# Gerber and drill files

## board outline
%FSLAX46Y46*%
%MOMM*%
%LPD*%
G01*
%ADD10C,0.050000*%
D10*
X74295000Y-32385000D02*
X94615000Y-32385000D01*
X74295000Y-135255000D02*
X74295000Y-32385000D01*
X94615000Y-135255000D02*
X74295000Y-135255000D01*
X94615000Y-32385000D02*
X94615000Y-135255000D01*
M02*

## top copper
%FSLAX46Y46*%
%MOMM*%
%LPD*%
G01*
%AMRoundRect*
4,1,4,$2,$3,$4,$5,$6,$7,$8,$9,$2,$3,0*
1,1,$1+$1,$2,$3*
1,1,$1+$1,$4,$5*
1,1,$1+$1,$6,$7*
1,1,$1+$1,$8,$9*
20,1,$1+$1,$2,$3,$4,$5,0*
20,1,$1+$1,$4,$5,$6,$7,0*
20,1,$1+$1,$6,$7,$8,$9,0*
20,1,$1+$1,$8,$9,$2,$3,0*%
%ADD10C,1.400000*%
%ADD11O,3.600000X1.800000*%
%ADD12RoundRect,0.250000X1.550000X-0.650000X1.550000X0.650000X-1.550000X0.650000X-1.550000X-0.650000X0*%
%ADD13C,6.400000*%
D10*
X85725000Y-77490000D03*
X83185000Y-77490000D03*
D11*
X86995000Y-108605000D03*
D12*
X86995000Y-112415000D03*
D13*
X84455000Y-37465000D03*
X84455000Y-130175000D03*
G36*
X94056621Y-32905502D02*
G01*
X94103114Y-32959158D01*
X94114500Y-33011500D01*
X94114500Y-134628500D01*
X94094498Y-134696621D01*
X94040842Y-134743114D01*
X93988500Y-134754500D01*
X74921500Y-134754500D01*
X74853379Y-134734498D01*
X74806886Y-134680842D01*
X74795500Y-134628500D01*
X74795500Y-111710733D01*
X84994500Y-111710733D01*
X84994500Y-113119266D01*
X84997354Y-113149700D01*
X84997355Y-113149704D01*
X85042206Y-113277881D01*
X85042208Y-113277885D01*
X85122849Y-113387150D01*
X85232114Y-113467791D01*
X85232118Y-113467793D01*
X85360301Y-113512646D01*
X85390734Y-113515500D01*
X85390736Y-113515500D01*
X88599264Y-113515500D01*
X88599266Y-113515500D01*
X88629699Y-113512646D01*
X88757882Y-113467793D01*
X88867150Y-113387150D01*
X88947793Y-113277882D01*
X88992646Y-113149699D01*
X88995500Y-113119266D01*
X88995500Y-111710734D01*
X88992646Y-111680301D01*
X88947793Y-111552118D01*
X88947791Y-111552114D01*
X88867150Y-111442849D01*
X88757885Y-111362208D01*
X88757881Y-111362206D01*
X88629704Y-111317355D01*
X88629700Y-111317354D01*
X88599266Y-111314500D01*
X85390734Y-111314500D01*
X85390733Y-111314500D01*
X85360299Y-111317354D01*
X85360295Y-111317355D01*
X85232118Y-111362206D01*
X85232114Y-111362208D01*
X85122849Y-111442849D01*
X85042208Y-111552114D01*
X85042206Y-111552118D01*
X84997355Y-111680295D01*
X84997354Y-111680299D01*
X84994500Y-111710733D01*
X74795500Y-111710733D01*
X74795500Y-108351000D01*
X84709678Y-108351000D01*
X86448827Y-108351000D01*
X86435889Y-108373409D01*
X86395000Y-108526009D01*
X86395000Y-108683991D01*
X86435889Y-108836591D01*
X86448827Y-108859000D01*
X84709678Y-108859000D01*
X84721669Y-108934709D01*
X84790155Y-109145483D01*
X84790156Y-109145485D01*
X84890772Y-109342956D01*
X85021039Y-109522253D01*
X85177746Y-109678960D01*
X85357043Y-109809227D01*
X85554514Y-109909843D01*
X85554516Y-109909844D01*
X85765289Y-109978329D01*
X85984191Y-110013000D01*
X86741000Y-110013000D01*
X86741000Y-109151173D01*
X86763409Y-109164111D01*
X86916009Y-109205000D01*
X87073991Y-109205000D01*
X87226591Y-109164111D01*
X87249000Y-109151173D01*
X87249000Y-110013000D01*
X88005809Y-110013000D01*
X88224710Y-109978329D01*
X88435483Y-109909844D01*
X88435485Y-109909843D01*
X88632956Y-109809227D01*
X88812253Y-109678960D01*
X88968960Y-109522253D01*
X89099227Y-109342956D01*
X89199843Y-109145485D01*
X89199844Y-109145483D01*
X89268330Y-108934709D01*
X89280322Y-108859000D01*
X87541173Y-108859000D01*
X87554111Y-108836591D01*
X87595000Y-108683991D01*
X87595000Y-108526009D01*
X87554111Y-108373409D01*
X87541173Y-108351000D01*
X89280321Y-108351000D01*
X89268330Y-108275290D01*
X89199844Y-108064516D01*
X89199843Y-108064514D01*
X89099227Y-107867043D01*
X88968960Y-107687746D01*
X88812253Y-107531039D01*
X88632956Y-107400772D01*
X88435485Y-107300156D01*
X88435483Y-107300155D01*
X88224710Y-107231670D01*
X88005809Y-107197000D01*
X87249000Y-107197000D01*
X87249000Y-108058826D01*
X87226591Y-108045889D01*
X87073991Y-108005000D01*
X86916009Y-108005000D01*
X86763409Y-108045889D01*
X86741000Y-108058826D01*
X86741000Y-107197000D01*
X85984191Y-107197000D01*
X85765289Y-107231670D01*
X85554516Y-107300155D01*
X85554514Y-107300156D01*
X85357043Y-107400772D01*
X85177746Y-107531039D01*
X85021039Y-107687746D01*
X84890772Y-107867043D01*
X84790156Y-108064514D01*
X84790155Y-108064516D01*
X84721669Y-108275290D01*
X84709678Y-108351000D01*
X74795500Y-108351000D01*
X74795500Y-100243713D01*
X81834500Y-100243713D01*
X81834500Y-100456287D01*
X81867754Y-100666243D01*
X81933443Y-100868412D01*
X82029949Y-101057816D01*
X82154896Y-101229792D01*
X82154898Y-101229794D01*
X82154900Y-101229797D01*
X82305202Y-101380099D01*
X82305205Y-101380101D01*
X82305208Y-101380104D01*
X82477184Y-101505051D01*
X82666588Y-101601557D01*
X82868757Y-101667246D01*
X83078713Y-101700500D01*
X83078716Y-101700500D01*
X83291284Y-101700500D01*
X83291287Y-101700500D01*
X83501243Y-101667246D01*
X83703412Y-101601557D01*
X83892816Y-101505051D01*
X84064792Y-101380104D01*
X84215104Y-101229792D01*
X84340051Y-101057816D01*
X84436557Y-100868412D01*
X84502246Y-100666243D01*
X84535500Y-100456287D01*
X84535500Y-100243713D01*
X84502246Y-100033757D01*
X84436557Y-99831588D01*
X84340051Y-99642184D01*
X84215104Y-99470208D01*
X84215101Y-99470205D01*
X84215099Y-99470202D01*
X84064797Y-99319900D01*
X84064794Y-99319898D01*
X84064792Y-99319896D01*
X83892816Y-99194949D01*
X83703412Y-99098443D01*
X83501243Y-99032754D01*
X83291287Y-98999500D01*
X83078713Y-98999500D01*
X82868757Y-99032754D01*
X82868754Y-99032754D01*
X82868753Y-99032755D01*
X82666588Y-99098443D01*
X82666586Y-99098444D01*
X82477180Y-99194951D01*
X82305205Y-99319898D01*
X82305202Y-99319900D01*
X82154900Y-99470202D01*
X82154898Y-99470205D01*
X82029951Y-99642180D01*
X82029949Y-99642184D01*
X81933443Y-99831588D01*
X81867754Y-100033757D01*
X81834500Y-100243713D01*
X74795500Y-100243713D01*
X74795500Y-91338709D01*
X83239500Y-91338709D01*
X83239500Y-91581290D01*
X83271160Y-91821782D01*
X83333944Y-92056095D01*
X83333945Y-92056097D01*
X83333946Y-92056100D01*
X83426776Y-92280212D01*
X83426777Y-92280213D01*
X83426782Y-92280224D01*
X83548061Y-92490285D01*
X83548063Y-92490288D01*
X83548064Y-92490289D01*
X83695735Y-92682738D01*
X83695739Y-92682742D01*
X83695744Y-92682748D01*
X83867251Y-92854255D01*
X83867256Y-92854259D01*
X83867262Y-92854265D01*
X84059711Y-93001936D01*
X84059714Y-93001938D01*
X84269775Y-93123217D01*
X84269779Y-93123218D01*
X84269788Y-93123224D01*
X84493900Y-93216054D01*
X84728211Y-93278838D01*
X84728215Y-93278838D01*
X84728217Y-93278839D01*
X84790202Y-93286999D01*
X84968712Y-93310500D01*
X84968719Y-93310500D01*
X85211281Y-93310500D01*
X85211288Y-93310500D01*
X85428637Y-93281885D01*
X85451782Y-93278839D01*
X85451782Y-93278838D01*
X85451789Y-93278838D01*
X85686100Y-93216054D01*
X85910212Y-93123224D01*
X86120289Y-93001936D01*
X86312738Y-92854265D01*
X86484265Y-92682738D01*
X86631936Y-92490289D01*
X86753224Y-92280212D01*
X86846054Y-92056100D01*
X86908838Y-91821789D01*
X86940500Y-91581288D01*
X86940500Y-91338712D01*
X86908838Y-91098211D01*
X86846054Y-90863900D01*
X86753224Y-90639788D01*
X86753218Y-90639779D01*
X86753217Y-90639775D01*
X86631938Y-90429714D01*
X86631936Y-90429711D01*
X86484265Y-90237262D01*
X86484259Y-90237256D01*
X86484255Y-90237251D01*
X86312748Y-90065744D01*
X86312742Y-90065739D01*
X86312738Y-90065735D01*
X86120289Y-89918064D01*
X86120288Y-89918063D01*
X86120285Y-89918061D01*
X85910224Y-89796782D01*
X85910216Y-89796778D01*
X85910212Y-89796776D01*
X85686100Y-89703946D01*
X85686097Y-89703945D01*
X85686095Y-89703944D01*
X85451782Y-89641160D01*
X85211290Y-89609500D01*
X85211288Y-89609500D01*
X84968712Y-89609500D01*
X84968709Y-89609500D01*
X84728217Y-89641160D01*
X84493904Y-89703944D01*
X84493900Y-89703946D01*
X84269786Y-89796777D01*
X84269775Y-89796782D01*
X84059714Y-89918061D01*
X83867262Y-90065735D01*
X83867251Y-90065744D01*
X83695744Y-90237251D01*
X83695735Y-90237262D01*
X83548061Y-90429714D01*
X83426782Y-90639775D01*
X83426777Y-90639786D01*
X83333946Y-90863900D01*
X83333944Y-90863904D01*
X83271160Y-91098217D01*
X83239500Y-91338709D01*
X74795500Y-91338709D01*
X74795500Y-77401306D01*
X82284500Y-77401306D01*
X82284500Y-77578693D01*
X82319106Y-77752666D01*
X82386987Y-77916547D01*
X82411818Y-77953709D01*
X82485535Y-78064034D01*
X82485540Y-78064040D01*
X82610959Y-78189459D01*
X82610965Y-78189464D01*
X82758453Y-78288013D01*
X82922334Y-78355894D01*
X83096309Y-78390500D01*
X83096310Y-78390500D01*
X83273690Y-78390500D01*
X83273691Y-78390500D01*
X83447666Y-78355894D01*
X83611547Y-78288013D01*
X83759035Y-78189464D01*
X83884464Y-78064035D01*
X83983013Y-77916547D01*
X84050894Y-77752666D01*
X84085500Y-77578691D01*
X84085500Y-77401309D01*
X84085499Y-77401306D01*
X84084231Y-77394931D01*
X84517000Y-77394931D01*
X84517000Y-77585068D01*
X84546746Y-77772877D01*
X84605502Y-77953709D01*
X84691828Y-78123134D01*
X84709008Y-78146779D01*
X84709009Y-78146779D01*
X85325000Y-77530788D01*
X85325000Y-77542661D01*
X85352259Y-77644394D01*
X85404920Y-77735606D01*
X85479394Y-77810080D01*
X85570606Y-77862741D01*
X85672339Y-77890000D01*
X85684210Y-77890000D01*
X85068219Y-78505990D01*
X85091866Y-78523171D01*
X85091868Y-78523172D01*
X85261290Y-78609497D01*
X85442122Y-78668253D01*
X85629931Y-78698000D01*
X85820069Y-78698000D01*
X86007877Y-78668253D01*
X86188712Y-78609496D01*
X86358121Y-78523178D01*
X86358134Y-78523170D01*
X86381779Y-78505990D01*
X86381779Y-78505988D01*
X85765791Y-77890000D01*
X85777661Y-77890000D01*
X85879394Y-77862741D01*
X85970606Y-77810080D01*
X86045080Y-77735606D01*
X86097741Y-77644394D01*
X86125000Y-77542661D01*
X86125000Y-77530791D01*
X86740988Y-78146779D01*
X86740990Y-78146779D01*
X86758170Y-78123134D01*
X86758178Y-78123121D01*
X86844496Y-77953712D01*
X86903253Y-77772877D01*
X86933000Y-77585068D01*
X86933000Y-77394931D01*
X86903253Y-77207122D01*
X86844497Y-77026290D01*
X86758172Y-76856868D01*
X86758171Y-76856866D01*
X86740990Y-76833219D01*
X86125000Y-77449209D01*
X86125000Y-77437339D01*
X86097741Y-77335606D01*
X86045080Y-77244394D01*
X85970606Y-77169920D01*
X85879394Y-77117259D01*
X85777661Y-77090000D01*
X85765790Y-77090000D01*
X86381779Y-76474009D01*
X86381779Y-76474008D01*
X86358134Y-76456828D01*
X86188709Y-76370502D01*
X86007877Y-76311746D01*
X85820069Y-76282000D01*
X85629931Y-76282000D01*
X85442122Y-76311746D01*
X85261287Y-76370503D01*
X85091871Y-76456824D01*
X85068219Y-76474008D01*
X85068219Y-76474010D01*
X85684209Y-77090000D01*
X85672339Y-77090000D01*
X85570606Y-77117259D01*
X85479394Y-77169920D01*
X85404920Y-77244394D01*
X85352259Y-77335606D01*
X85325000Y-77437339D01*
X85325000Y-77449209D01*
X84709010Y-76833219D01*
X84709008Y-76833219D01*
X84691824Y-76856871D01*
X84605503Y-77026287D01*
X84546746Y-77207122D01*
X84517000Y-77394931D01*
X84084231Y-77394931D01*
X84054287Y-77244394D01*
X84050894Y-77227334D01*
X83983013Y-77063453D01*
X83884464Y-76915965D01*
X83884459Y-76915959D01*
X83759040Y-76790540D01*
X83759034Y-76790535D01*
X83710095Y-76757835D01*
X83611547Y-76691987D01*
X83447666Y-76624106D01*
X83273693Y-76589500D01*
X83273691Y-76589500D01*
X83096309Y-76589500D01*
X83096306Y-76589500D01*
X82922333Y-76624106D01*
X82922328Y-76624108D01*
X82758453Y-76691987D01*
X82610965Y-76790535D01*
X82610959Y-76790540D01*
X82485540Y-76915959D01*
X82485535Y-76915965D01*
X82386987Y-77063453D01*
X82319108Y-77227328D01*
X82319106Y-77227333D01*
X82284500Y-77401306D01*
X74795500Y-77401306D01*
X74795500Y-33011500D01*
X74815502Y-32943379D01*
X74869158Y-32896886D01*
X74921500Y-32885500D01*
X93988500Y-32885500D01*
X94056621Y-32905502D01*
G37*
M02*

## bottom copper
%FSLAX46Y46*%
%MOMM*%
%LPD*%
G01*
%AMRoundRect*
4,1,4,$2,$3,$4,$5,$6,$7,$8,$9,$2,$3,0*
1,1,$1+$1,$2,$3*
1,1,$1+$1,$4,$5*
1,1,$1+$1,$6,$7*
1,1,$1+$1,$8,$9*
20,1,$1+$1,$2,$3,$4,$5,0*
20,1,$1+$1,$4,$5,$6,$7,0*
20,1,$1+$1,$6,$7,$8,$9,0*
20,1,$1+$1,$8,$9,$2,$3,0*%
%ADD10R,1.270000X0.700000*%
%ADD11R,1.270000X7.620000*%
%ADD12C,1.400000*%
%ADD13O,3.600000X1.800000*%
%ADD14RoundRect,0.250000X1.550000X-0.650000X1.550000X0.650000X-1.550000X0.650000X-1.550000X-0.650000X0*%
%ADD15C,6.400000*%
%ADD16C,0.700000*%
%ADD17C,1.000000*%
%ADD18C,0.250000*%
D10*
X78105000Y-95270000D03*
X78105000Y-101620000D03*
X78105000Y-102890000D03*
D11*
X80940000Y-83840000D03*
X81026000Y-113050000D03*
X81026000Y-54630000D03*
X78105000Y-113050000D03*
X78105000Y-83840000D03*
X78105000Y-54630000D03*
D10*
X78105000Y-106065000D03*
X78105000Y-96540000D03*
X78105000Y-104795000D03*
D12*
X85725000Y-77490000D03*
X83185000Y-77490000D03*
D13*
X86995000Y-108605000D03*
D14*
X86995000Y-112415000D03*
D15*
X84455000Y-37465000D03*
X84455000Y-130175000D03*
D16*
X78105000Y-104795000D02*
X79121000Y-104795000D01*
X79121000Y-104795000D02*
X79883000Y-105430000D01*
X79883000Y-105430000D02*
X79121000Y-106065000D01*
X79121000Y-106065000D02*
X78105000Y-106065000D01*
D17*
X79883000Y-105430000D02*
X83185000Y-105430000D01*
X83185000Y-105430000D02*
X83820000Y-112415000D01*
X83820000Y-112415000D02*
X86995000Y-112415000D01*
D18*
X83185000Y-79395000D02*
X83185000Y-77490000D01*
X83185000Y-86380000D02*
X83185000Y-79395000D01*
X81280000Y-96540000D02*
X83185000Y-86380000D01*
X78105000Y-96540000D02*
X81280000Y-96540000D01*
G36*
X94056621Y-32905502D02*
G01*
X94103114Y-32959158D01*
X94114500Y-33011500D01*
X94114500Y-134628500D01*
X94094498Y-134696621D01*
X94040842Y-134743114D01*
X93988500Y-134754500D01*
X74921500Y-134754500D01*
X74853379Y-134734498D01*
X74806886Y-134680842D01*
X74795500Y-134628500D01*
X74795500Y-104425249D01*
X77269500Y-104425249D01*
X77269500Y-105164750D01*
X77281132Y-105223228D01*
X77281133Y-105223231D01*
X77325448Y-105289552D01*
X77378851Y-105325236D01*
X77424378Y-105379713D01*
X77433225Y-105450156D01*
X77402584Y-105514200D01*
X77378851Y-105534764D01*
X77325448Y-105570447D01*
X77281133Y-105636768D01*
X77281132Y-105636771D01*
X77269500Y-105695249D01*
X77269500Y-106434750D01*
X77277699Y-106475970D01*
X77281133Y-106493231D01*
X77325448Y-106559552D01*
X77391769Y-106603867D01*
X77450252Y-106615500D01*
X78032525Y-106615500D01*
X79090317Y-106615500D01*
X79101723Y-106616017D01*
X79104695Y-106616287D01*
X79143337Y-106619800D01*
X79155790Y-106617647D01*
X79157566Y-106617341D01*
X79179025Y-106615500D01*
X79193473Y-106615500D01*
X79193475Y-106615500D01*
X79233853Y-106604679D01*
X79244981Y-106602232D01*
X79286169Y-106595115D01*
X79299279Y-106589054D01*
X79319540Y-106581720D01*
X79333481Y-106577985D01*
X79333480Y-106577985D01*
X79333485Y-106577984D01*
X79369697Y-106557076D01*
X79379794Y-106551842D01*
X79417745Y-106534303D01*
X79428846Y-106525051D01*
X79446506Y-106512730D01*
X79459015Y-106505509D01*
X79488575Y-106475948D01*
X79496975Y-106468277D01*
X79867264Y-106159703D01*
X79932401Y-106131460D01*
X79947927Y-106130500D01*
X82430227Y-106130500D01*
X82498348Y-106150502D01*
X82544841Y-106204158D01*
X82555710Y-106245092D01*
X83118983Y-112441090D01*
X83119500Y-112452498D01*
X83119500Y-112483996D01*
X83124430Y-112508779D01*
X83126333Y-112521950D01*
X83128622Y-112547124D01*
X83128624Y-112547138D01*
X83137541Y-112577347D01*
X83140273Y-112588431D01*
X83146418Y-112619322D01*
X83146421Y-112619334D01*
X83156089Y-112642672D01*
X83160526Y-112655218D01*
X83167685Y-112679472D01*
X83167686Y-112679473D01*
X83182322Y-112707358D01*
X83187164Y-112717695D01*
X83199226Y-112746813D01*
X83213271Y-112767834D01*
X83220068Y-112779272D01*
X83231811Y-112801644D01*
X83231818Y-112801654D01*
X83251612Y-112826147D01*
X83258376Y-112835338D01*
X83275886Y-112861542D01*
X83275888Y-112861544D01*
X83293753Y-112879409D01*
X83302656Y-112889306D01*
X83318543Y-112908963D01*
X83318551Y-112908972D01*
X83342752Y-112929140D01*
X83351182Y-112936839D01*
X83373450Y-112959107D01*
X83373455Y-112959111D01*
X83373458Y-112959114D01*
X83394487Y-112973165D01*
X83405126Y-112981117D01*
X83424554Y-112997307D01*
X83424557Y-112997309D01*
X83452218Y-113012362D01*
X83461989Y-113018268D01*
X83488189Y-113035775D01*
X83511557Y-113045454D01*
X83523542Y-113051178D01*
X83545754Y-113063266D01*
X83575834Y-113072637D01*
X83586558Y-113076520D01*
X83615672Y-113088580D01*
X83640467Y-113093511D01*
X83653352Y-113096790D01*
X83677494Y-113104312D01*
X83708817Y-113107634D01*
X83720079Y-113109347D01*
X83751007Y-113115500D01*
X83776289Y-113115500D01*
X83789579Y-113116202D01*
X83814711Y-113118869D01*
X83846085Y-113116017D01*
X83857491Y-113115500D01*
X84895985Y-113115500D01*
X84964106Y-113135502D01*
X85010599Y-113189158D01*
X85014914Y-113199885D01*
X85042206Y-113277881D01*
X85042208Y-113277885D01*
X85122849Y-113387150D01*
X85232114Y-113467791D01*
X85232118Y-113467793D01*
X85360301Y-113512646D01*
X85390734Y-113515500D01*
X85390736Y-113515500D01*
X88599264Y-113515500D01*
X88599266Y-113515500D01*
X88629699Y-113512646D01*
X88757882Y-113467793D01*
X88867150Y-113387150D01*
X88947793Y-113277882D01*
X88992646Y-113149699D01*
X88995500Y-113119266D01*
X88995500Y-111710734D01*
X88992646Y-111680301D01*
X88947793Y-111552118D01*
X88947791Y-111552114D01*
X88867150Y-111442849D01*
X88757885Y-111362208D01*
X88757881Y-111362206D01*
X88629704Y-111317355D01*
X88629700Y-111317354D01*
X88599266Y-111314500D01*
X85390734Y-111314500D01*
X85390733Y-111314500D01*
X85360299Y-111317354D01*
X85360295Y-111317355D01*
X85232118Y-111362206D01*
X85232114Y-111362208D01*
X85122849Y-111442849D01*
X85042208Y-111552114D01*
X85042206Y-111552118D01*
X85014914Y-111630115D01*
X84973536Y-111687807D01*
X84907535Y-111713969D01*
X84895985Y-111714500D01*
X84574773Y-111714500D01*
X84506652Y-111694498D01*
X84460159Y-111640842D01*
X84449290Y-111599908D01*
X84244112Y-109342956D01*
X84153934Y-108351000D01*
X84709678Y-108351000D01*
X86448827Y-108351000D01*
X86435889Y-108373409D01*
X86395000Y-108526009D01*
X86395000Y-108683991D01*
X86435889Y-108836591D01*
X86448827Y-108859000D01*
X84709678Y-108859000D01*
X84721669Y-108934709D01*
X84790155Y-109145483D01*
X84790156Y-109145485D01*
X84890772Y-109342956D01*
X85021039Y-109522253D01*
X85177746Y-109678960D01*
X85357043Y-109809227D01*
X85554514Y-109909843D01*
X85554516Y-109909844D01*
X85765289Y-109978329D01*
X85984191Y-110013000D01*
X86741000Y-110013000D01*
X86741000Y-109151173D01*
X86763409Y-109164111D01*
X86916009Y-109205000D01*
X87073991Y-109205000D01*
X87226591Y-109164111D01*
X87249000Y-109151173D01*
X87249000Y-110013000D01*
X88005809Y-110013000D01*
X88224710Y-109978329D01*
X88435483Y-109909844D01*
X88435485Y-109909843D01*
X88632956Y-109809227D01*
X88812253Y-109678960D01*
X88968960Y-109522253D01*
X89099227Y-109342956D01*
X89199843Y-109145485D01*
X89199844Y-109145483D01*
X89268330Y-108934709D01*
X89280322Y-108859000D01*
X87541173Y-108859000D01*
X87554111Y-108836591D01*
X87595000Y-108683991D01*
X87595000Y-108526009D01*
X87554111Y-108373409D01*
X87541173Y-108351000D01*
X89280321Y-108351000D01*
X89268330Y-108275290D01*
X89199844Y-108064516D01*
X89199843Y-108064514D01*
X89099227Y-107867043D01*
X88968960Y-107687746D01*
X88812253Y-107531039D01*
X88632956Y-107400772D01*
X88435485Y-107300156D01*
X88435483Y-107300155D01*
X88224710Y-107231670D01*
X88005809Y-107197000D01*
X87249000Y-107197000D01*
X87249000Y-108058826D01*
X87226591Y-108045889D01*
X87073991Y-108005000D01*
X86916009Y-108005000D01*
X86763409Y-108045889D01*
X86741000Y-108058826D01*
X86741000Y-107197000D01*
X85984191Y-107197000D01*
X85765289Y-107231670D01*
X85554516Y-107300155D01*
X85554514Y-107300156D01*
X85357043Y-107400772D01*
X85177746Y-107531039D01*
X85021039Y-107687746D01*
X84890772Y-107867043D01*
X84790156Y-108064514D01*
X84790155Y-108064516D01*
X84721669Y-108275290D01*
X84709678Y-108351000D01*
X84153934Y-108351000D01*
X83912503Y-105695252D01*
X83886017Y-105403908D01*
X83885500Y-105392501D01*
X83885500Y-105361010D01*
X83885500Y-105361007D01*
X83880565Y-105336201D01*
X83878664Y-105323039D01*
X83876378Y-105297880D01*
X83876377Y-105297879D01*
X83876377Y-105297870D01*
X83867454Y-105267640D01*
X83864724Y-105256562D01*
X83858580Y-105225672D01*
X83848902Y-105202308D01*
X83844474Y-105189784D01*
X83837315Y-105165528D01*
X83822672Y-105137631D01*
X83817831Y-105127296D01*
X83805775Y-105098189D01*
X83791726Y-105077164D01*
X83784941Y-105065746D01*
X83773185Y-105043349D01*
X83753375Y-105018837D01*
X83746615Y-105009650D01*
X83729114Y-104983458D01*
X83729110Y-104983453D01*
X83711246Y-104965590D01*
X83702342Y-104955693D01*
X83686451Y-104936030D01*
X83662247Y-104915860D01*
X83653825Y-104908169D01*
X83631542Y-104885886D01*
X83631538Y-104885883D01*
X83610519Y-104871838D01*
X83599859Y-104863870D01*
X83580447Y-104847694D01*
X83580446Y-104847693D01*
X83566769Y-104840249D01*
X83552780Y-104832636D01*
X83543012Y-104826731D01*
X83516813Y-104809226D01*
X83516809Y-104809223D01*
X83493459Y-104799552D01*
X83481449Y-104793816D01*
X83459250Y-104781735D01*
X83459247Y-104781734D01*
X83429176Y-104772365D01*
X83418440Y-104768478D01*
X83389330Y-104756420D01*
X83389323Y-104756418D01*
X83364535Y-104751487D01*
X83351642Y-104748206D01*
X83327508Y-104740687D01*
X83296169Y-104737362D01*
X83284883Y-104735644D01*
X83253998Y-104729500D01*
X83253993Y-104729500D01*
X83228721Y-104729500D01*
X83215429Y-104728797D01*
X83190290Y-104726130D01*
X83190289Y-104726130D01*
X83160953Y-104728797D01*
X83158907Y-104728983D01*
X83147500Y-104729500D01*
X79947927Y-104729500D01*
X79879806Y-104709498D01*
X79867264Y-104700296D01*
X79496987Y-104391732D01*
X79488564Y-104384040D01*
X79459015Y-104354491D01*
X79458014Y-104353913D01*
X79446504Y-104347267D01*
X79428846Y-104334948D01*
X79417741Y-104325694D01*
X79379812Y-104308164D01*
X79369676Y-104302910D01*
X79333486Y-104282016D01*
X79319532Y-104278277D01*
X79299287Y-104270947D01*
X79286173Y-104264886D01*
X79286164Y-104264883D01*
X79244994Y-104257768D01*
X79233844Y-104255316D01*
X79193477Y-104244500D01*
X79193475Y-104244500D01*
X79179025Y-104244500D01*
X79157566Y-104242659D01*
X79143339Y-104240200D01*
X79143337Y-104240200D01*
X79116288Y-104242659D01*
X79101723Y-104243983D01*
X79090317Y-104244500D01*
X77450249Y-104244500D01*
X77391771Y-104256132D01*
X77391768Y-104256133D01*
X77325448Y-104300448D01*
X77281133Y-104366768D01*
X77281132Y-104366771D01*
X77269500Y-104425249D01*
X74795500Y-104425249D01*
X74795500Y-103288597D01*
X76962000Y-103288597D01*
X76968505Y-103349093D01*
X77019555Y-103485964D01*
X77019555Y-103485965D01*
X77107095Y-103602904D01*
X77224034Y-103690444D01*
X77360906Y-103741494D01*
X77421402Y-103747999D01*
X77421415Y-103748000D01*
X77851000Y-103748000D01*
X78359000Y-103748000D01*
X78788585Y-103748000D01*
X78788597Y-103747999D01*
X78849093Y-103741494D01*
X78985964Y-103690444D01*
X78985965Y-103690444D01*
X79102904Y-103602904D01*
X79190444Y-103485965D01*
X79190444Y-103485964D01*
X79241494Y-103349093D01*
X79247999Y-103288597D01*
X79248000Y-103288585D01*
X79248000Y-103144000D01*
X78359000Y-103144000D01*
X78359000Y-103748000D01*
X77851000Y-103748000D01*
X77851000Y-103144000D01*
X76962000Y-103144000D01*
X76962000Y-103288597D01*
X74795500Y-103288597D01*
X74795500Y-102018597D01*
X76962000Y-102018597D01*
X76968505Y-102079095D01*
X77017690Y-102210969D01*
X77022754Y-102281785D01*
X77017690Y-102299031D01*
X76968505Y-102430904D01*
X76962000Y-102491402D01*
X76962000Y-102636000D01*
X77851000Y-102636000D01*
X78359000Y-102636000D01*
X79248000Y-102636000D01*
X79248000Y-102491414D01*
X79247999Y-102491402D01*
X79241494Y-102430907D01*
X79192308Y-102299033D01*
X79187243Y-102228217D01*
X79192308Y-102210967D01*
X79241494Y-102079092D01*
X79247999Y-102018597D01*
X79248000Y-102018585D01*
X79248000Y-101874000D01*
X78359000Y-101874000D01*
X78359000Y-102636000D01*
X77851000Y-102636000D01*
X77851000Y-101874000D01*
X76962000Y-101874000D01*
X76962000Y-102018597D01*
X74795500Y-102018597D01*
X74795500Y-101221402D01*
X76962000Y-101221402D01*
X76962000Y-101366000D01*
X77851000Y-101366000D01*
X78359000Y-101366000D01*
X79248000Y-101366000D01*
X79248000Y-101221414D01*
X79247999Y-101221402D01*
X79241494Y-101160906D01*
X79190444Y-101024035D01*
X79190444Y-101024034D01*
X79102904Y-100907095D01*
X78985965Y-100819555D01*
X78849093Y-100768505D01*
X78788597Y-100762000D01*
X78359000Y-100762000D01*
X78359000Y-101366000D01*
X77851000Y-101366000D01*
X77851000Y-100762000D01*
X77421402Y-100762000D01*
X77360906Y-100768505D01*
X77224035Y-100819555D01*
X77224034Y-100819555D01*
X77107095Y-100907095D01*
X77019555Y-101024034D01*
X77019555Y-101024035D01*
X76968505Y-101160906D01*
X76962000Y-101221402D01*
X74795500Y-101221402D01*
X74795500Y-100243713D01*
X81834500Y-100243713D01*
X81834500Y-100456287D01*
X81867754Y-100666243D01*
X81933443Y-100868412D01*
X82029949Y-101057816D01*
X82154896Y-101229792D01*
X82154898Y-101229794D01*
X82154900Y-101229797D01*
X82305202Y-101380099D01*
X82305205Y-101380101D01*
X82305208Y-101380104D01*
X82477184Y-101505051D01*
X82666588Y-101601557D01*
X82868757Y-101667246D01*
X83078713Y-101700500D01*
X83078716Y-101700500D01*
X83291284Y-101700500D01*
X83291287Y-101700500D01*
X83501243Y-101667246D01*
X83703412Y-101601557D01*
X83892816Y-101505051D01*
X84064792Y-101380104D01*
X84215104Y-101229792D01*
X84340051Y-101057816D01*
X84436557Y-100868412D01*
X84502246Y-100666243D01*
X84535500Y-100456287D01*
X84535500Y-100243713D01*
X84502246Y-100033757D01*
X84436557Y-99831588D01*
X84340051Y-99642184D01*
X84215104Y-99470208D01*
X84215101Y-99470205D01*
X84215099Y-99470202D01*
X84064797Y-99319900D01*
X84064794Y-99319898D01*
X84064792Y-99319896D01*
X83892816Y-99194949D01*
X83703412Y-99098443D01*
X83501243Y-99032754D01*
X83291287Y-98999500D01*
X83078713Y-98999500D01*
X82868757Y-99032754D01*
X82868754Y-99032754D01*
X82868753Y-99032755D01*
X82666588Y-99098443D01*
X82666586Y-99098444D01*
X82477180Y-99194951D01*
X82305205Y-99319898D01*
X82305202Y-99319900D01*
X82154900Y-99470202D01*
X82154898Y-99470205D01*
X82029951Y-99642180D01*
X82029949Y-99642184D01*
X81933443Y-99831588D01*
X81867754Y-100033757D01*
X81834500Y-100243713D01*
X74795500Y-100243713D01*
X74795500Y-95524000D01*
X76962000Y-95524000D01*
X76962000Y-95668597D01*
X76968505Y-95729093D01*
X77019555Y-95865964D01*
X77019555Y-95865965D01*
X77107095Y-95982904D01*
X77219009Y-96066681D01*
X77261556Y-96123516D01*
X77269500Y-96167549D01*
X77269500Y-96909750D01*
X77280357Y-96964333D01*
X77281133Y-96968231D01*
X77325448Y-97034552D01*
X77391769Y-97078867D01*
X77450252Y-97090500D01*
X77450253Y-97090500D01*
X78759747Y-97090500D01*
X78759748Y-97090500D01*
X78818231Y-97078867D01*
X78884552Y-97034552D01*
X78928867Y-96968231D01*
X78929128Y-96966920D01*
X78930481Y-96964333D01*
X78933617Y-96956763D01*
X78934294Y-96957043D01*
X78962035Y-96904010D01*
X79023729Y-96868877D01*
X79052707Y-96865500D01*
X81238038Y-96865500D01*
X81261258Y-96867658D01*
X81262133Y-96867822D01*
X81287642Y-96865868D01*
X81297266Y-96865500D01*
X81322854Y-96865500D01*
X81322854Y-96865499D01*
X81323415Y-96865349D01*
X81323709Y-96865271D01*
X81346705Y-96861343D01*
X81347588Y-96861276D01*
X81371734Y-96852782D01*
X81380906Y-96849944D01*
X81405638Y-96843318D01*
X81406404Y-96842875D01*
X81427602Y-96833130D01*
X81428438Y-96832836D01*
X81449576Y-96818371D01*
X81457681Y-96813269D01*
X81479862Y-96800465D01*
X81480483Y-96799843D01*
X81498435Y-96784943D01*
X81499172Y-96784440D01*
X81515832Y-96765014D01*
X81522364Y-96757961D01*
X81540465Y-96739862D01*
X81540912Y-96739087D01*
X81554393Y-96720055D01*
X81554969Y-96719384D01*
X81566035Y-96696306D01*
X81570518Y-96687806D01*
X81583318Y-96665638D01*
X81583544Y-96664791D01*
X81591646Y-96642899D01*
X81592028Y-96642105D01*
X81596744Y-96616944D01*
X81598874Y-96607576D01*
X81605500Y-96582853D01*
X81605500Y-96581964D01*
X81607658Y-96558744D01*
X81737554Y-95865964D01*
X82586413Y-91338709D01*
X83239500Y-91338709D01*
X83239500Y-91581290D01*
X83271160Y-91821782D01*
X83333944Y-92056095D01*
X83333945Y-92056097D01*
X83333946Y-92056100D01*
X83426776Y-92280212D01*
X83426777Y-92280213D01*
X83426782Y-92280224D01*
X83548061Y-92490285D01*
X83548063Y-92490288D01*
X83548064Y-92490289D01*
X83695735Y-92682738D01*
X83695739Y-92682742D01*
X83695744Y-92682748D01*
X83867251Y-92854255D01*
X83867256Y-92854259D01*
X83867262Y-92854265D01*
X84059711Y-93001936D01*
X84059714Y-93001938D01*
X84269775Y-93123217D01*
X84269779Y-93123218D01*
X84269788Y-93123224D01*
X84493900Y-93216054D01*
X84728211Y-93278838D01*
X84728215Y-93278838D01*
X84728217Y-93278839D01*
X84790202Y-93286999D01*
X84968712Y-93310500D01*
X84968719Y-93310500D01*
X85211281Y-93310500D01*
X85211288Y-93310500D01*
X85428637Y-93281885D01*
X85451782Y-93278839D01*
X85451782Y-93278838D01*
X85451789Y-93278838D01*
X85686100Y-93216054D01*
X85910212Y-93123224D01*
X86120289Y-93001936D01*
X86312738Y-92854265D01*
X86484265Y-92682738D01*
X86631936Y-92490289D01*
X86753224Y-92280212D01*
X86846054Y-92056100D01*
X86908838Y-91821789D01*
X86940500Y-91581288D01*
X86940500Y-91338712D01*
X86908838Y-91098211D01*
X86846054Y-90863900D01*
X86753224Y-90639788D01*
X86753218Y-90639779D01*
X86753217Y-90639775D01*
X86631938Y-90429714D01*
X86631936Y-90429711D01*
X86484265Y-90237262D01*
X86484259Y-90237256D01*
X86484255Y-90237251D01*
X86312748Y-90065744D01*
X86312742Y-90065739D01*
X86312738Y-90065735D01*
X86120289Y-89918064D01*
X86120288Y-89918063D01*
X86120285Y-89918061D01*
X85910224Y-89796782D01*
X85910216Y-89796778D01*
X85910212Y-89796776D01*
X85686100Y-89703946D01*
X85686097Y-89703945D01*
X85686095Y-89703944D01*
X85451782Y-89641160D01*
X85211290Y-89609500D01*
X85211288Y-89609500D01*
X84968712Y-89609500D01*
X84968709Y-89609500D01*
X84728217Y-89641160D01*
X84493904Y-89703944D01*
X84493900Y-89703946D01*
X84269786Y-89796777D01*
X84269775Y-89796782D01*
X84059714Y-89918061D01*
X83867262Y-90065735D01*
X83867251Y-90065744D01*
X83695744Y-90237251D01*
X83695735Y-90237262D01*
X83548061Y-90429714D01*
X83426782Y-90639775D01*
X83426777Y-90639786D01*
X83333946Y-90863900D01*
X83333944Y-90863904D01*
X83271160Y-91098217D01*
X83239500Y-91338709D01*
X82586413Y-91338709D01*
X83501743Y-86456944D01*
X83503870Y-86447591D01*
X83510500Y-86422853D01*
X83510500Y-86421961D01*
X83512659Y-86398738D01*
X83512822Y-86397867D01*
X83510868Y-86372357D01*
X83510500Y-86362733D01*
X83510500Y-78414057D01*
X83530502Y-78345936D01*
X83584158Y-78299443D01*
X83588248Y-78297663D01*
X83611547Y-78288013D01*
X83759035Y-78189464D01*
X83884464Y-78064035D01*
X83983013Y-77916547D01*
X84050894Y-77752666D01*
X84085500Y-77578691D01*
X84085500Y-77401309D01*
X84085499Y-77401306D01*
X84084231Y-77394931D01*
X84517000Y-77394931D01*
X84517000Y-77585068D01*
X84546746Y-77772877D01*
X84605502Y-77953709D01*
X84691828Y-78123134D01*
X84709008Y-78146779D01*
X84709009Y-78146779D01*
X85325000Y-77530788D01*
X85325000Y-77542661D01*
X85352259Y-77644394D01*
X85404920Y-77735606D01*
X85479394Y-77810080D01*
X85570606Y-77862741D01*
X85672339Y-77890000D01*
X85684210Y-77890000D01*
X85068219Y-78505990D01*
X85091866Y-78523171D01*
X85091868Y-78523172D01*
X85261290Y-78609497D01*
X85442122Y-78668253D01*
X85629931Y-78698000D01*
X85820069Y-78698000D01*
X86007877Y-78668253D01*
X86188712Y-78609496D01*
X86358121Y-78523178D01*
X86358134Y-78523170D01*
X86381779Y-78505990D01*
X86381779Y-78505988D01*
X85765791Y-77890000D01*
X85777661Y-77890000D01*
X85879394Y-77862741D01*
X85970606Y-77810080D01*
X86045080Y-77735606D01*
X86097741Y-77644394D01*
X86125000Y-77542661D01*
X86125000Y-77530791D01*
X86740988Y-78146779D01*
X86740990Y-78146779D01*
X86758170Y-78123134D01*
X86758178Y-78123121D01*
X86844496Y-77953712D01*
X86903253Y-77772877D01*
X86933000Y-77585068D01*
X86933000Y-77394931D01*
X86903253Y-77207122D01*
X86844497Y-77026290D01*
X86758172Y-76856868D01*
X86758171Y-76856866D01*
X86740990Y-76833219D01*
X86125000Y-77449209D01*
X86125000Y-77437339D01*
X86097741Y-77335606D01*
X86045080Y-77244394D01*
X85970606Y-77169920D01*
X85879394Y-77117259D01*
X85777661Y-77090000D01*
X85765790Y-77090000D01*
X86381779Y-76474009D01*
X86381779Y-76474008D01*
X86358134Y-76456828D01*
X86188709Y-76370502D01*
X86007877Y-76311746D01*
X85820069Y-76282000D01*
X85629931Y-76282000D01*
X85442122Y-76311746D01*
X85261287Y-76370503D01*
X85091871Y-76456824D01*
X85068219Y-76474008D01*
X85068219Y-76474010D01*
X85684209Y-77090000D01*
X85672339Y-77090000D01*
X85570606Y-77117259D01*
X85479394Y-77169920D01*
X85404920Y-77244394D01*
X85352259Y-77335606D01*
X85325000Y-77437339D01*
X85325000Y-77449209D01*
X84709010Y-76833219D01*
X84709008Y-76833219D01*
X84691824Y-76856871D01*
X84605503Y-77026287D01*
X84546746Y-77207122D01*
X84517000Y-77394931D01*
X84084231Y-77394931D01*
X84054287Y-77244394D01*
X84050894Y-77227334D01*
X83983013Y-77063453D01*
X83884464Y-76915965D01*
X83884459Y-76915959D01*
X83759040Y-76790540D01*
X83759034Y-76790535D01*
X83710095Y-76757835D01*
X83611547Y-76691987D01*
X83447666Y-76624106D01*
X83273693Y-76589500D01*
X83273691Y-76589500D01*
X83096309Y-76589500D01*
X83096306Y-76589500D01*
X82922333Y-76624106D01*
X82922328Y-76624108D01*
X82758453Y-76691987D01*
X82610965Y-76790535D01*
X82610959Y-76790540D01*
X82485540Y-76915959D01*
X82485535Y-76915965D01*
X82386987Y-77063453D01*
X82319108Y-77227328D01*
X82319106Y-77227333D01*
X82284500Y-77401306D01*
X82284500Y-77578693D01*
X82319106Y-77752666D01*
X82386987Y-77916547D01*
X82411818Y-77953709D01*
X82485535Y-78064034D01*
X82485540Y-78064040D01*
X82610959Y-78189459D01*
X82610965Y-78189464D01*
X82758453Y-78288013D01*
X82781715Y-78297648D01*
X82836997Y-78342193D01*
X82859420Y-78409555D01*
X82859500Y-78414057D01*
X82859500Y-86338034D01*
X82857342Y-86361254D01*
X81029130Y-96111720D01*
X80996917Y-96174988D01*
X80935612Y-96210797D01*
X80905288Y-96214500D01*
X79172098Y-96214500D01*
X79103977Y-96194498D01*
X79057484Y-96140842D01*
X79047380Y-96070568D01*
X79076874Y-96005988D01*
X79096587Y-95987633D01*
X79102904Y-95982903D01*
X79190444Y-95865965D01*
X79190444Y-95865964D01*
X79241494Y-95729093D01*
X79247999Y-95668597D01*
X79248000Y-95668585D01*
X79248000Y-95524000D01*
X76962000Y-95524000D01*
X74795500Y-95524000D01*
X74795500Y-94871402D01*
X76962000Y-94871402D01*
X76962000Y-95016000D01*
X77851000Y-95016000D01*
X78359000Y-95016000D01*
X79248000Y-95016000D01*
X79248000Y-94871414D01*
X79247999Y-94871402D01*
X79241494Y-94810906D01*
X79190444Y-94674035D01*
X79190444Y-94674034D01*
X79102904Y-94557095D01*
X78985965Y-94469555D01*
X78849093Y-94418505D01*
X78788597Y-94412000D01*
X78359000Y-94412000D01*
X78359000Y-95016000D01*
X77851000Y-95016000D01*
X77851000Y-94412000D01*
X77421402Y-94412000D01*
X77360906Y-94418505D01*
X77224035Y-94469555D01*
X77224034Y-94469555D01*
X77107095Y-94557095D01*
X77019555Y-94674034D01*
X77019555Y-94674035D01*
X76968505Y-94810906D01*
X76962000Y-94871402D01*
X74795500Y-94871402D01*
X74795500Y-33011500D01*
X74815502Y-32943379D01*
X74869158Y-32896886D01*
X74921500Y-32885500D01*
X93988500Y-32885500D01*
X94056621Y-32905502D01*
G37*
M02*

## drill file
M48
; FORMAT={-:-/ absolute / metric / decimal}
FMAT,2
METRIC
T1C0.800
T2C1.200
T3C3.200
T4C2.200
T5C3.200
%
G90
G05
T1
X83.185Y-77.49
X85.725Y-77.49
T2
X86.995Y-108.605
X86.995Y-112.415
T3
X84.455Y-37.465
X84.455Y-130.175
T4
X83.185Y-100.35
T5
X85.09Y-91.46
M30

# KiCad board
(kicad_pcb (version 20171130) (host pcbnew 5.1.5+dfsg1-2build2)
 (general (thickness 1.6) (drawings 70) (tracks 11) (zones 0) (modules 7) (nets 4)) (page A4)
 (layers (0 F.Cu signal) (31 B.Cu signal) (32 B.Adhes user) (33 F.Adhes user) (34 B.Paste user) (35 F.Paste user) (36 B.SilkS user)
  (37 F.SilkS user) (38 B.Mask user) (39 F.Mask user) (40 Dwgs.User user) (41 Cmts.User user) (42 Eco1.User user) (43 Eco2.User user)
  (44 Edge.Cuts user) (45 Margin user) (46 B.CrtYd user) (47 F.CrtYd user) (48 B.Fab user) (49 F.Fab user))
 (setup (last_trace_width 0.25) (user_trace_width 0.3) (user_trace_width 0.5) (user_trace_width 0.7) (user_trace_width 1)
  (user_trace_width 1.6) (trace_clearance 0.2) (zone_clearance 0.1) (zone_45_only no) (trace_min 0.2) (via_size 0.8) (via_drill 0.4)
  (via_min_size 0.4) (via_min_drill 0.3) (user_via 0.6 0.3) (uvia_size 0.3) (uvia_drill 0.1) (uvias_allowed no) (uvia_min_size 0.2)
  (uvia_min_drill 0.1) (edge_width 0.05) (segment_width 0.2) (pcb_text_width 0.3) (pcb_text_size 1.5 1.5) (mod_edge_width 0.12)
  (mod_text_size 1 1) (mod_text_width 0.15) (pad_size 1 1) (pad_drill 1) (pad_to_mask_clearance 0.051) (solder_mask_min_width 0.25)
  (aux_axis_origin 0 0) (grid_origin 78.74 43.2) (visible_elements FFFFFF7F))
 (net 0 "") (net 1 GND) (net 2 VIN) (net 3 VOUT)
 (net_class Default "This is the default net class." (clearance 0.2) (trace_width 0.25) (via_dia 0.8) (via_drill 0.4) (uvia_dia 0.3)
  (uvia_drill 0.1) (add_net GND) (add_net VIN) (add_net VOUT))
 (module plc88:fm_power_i (layer F.Cu) (at 80.645 55.265)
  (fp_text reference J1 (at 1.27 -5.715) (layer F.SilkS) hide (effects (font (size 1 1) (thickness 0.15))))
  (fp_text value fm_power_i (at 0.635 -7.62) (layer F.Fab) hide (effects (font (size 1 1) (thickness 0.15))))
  (pad 4 smd rect (at -2.54 40.005) (size 1.27 0.7) (layers B.Cu B.Paste B.Mask) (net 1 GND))
  (pad 2 smd rect (at -2.54 46.355) (size 1.27 0.7) (layers B.Cu B.Paste B.Mask) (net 1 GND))
  (pad 2 smd rect (at -2.54 47.625) (size 1.27 0.7) (layers B.Cu B.Paste B.Mask) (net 1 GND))
  (pad 5 smd rect (at 0.295 28.575) (size 1.27 7.62) (layers B.Cu B.Paste B.Mask) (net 1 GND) (zone_connect 2))
  (pad 5 smd rect (at 0.381 57.785) (size 1.27 7.62) (layers B.Cu B.Paste B.Mask) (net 1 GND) (zone_connect 2))
  (pad 5 smd rect (at 0.381 -0.635) (size 1.27 7.62) (layers B.Cu B.Paste B.Mask) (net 1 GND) (zone_connect 2))
  (pad 5 smd rect (at -2.54 57.785) (size 1.27 7.62) (layers B.Cu B.Paste B.Mask) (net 1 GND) (zone_connect 2))
  (pad 5 smd rect (at -2.54 28.575) (size 1.27 7.62) (layers B.Cu B.Paste B.Mask) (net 1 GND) (zone_connect 2))
  (pad 5 smd rect (at -2.54 -0.635) (size 1.27 7.62) (layers B.Cu B.Paste B.Mask) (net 1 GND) (zone_connect 2))
  (pad 1 smd rect (at -2.54 50.8) (size 1.27 0.7) (layers B.Cu B.Paste B.Mask) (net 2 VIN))
  (pad 3 smd rect (at -2.54 41.275) (size 1.27 0.7) (layers B.Cu B.Paste B.Mask) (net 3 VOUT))
  (pad 1 smd rect (at -2.54 49.53) (size 1.27 0.7) (layers B.Cu B.Paste B.Mask) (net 2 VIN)))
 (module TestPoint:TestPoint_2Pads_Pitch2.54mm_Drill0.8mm (layer F.Cu) (at 83.185 77.49)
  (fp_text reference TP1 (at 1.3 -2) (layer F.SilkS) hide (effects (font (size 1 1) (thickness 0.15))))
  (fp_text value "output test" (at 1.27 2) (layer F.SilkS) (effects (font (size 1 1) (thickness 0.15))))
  (pad 2 thru_hole circle (at 2.54 0) (size 1.4 1.4) (drill 0.8) (layers *.Cu *.Mask) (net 1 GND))
  (pad 1 thru_hole circle (at 0 0) (size 1.4 1.4) (drill 0.8) (layers *.Cu *.Mask) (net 3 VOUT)))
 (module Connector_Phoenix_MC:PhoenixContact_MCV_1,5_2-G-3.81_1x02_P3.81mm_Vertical (layer F.Cu) (at 86.995 112.415 90)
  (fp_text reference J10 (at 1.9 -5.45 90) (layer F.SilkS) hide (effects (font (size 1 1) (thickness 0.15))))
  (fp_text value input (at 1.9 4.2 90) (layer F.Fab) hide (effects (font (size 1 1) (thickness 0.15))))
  (pad 2 thru_hole oval (at 3.81 0 90) (size 1.8 3.6) (drill 1.2) (layers *.Cu *.Mask) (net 1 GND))
  (pad 1 thru_hole roundrect (at 0 0 90) (size 1.8 3.6) (drill 1.2) (layers *.Cu *.Mask) (roundrect_rratio 0.138889) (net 2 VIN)))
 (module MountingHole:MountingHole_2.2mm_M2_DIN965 (layer F.Cu) (at 83.185 100.35)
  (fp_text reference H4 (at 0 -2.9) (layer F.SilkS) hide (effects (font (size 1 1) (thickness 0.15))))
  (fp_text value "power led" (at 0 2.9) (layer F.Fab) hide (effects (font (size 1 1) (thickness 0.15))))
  (pad 1 np_thru_hole circle (at 0 0) (size 2.2 2.2) (drill 2.2) (layers *.Cu *.Mask)))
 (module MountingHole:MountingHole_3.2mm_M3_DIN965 (layer F.Cu) (at 85.09 91.46)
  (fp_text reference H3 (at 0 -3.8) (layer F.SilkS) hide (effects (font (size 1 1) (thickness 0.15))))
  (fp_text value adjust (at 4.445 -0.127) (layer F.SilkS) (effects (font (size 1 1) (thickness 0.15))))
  (pad 1 np_thru_hole circle (at 0 0) (size 3.2 3.2) (drill 3.2) (layers *.Cu *.Mask)))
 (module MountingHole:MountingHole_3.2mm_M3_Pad (layer F.Cu) (at 84.455 37.465)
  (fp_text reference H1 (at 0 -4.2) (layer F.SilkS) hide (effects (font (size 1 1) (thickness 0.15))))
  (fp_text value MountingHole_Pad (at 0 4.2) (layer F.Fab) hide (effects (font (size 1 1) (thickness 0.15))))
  (pad 1 thru_hole circle (at 0 0) (size 6.4 6.4) (drill 3.2) (layers *.Cu *.Mask) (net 1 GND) (zone_connect 2)))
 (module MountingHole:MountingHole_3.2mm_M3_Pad (layer F.Cu) (at 84.455 130.175)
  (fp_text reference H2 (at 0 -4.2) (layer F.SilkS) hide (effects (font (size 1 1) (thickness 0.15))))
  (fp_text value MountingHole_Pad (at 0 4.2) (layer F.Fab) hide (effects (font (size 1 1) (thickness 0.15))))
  (pad 1 thru_hole circle (at 0 0) (size 6.4 6.4) (drill 3.2) (layers *.Cu *.Mask) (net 1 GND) (zone_connect 2)))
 (gr_line (start 74.295 32.385) (end 94.615 32.385) (layer Edge.Cuts) (width 0.05))
 (gr_line (start 74.295 135.255) (end 74.295 32.385) (layer Edge.Cuts) (width 0.05))
 (gr_line (start 94.615 135.255) (end 74.295 135.255) (layer Edge.Cuts) (width 0.05))
 (gr_line (start 94.615 32.385) (end 94.615 135.255) (layer Edge.Cuts) (width 0.05))
 (segment (start 78.105 104.795) (end 79.121 104.795) (width 0.7) (layer B.Cu) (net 2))
 (segment (start 79.121 104.795) (end 79.883 105.43) (width 0.7) (layer B.Cu) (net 2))
 (segment (start 79.883 105.43) (end 79.121 106.065) (width 0.7) (layer B.Cu) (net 2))
 (segment (start 79.121 106.065) (end 78.105 106.065) (width 0.7) (layer B.Cu) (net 2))
 (segment (start 79.883 105.43) (end 83.185 105.43) (width 1) (layer B.Cu) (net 2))
 (segment (start 83.185 105.43) (end 83.82 112.415) (width 1) (layer B.Cu) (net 2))
 (segment (start 83.82 112.415) (end 86.995 112.415) (width 1) (layer B.Cu) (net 2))
 (segment (start 83.185 79.395) (end 83.185 77.49) (width 0.25) (layer B.Cu) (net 3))
 (segment (start 83.185 86.38) (end 83.185 79.395) (width 0.25) (layer B.Cu) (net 3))
 (segment (start 81.28 96.54) (end 83.185 86.38) (width 0.25) (layer B.Cu) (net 3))
 (segment (start 78.105 96.54) (end 81.28 96.54) (width 0.25) (layer B.Cu) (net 3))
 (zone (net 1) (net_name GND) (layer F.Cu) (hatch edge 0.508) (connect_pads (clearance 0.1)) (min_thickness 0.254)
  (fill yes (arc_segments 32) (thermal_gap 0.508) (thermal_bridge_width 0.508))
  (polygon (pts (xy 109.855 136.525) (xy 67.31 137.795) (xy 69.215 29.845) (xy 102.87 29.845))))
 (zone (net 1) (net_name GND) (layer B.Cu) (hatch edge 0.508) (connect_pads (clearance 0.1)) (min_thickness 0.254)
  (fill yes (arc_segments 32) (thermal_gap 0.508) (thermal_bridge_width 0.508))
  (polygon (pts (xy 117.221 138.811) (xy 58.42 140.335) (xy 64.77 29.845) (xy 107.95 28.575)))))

